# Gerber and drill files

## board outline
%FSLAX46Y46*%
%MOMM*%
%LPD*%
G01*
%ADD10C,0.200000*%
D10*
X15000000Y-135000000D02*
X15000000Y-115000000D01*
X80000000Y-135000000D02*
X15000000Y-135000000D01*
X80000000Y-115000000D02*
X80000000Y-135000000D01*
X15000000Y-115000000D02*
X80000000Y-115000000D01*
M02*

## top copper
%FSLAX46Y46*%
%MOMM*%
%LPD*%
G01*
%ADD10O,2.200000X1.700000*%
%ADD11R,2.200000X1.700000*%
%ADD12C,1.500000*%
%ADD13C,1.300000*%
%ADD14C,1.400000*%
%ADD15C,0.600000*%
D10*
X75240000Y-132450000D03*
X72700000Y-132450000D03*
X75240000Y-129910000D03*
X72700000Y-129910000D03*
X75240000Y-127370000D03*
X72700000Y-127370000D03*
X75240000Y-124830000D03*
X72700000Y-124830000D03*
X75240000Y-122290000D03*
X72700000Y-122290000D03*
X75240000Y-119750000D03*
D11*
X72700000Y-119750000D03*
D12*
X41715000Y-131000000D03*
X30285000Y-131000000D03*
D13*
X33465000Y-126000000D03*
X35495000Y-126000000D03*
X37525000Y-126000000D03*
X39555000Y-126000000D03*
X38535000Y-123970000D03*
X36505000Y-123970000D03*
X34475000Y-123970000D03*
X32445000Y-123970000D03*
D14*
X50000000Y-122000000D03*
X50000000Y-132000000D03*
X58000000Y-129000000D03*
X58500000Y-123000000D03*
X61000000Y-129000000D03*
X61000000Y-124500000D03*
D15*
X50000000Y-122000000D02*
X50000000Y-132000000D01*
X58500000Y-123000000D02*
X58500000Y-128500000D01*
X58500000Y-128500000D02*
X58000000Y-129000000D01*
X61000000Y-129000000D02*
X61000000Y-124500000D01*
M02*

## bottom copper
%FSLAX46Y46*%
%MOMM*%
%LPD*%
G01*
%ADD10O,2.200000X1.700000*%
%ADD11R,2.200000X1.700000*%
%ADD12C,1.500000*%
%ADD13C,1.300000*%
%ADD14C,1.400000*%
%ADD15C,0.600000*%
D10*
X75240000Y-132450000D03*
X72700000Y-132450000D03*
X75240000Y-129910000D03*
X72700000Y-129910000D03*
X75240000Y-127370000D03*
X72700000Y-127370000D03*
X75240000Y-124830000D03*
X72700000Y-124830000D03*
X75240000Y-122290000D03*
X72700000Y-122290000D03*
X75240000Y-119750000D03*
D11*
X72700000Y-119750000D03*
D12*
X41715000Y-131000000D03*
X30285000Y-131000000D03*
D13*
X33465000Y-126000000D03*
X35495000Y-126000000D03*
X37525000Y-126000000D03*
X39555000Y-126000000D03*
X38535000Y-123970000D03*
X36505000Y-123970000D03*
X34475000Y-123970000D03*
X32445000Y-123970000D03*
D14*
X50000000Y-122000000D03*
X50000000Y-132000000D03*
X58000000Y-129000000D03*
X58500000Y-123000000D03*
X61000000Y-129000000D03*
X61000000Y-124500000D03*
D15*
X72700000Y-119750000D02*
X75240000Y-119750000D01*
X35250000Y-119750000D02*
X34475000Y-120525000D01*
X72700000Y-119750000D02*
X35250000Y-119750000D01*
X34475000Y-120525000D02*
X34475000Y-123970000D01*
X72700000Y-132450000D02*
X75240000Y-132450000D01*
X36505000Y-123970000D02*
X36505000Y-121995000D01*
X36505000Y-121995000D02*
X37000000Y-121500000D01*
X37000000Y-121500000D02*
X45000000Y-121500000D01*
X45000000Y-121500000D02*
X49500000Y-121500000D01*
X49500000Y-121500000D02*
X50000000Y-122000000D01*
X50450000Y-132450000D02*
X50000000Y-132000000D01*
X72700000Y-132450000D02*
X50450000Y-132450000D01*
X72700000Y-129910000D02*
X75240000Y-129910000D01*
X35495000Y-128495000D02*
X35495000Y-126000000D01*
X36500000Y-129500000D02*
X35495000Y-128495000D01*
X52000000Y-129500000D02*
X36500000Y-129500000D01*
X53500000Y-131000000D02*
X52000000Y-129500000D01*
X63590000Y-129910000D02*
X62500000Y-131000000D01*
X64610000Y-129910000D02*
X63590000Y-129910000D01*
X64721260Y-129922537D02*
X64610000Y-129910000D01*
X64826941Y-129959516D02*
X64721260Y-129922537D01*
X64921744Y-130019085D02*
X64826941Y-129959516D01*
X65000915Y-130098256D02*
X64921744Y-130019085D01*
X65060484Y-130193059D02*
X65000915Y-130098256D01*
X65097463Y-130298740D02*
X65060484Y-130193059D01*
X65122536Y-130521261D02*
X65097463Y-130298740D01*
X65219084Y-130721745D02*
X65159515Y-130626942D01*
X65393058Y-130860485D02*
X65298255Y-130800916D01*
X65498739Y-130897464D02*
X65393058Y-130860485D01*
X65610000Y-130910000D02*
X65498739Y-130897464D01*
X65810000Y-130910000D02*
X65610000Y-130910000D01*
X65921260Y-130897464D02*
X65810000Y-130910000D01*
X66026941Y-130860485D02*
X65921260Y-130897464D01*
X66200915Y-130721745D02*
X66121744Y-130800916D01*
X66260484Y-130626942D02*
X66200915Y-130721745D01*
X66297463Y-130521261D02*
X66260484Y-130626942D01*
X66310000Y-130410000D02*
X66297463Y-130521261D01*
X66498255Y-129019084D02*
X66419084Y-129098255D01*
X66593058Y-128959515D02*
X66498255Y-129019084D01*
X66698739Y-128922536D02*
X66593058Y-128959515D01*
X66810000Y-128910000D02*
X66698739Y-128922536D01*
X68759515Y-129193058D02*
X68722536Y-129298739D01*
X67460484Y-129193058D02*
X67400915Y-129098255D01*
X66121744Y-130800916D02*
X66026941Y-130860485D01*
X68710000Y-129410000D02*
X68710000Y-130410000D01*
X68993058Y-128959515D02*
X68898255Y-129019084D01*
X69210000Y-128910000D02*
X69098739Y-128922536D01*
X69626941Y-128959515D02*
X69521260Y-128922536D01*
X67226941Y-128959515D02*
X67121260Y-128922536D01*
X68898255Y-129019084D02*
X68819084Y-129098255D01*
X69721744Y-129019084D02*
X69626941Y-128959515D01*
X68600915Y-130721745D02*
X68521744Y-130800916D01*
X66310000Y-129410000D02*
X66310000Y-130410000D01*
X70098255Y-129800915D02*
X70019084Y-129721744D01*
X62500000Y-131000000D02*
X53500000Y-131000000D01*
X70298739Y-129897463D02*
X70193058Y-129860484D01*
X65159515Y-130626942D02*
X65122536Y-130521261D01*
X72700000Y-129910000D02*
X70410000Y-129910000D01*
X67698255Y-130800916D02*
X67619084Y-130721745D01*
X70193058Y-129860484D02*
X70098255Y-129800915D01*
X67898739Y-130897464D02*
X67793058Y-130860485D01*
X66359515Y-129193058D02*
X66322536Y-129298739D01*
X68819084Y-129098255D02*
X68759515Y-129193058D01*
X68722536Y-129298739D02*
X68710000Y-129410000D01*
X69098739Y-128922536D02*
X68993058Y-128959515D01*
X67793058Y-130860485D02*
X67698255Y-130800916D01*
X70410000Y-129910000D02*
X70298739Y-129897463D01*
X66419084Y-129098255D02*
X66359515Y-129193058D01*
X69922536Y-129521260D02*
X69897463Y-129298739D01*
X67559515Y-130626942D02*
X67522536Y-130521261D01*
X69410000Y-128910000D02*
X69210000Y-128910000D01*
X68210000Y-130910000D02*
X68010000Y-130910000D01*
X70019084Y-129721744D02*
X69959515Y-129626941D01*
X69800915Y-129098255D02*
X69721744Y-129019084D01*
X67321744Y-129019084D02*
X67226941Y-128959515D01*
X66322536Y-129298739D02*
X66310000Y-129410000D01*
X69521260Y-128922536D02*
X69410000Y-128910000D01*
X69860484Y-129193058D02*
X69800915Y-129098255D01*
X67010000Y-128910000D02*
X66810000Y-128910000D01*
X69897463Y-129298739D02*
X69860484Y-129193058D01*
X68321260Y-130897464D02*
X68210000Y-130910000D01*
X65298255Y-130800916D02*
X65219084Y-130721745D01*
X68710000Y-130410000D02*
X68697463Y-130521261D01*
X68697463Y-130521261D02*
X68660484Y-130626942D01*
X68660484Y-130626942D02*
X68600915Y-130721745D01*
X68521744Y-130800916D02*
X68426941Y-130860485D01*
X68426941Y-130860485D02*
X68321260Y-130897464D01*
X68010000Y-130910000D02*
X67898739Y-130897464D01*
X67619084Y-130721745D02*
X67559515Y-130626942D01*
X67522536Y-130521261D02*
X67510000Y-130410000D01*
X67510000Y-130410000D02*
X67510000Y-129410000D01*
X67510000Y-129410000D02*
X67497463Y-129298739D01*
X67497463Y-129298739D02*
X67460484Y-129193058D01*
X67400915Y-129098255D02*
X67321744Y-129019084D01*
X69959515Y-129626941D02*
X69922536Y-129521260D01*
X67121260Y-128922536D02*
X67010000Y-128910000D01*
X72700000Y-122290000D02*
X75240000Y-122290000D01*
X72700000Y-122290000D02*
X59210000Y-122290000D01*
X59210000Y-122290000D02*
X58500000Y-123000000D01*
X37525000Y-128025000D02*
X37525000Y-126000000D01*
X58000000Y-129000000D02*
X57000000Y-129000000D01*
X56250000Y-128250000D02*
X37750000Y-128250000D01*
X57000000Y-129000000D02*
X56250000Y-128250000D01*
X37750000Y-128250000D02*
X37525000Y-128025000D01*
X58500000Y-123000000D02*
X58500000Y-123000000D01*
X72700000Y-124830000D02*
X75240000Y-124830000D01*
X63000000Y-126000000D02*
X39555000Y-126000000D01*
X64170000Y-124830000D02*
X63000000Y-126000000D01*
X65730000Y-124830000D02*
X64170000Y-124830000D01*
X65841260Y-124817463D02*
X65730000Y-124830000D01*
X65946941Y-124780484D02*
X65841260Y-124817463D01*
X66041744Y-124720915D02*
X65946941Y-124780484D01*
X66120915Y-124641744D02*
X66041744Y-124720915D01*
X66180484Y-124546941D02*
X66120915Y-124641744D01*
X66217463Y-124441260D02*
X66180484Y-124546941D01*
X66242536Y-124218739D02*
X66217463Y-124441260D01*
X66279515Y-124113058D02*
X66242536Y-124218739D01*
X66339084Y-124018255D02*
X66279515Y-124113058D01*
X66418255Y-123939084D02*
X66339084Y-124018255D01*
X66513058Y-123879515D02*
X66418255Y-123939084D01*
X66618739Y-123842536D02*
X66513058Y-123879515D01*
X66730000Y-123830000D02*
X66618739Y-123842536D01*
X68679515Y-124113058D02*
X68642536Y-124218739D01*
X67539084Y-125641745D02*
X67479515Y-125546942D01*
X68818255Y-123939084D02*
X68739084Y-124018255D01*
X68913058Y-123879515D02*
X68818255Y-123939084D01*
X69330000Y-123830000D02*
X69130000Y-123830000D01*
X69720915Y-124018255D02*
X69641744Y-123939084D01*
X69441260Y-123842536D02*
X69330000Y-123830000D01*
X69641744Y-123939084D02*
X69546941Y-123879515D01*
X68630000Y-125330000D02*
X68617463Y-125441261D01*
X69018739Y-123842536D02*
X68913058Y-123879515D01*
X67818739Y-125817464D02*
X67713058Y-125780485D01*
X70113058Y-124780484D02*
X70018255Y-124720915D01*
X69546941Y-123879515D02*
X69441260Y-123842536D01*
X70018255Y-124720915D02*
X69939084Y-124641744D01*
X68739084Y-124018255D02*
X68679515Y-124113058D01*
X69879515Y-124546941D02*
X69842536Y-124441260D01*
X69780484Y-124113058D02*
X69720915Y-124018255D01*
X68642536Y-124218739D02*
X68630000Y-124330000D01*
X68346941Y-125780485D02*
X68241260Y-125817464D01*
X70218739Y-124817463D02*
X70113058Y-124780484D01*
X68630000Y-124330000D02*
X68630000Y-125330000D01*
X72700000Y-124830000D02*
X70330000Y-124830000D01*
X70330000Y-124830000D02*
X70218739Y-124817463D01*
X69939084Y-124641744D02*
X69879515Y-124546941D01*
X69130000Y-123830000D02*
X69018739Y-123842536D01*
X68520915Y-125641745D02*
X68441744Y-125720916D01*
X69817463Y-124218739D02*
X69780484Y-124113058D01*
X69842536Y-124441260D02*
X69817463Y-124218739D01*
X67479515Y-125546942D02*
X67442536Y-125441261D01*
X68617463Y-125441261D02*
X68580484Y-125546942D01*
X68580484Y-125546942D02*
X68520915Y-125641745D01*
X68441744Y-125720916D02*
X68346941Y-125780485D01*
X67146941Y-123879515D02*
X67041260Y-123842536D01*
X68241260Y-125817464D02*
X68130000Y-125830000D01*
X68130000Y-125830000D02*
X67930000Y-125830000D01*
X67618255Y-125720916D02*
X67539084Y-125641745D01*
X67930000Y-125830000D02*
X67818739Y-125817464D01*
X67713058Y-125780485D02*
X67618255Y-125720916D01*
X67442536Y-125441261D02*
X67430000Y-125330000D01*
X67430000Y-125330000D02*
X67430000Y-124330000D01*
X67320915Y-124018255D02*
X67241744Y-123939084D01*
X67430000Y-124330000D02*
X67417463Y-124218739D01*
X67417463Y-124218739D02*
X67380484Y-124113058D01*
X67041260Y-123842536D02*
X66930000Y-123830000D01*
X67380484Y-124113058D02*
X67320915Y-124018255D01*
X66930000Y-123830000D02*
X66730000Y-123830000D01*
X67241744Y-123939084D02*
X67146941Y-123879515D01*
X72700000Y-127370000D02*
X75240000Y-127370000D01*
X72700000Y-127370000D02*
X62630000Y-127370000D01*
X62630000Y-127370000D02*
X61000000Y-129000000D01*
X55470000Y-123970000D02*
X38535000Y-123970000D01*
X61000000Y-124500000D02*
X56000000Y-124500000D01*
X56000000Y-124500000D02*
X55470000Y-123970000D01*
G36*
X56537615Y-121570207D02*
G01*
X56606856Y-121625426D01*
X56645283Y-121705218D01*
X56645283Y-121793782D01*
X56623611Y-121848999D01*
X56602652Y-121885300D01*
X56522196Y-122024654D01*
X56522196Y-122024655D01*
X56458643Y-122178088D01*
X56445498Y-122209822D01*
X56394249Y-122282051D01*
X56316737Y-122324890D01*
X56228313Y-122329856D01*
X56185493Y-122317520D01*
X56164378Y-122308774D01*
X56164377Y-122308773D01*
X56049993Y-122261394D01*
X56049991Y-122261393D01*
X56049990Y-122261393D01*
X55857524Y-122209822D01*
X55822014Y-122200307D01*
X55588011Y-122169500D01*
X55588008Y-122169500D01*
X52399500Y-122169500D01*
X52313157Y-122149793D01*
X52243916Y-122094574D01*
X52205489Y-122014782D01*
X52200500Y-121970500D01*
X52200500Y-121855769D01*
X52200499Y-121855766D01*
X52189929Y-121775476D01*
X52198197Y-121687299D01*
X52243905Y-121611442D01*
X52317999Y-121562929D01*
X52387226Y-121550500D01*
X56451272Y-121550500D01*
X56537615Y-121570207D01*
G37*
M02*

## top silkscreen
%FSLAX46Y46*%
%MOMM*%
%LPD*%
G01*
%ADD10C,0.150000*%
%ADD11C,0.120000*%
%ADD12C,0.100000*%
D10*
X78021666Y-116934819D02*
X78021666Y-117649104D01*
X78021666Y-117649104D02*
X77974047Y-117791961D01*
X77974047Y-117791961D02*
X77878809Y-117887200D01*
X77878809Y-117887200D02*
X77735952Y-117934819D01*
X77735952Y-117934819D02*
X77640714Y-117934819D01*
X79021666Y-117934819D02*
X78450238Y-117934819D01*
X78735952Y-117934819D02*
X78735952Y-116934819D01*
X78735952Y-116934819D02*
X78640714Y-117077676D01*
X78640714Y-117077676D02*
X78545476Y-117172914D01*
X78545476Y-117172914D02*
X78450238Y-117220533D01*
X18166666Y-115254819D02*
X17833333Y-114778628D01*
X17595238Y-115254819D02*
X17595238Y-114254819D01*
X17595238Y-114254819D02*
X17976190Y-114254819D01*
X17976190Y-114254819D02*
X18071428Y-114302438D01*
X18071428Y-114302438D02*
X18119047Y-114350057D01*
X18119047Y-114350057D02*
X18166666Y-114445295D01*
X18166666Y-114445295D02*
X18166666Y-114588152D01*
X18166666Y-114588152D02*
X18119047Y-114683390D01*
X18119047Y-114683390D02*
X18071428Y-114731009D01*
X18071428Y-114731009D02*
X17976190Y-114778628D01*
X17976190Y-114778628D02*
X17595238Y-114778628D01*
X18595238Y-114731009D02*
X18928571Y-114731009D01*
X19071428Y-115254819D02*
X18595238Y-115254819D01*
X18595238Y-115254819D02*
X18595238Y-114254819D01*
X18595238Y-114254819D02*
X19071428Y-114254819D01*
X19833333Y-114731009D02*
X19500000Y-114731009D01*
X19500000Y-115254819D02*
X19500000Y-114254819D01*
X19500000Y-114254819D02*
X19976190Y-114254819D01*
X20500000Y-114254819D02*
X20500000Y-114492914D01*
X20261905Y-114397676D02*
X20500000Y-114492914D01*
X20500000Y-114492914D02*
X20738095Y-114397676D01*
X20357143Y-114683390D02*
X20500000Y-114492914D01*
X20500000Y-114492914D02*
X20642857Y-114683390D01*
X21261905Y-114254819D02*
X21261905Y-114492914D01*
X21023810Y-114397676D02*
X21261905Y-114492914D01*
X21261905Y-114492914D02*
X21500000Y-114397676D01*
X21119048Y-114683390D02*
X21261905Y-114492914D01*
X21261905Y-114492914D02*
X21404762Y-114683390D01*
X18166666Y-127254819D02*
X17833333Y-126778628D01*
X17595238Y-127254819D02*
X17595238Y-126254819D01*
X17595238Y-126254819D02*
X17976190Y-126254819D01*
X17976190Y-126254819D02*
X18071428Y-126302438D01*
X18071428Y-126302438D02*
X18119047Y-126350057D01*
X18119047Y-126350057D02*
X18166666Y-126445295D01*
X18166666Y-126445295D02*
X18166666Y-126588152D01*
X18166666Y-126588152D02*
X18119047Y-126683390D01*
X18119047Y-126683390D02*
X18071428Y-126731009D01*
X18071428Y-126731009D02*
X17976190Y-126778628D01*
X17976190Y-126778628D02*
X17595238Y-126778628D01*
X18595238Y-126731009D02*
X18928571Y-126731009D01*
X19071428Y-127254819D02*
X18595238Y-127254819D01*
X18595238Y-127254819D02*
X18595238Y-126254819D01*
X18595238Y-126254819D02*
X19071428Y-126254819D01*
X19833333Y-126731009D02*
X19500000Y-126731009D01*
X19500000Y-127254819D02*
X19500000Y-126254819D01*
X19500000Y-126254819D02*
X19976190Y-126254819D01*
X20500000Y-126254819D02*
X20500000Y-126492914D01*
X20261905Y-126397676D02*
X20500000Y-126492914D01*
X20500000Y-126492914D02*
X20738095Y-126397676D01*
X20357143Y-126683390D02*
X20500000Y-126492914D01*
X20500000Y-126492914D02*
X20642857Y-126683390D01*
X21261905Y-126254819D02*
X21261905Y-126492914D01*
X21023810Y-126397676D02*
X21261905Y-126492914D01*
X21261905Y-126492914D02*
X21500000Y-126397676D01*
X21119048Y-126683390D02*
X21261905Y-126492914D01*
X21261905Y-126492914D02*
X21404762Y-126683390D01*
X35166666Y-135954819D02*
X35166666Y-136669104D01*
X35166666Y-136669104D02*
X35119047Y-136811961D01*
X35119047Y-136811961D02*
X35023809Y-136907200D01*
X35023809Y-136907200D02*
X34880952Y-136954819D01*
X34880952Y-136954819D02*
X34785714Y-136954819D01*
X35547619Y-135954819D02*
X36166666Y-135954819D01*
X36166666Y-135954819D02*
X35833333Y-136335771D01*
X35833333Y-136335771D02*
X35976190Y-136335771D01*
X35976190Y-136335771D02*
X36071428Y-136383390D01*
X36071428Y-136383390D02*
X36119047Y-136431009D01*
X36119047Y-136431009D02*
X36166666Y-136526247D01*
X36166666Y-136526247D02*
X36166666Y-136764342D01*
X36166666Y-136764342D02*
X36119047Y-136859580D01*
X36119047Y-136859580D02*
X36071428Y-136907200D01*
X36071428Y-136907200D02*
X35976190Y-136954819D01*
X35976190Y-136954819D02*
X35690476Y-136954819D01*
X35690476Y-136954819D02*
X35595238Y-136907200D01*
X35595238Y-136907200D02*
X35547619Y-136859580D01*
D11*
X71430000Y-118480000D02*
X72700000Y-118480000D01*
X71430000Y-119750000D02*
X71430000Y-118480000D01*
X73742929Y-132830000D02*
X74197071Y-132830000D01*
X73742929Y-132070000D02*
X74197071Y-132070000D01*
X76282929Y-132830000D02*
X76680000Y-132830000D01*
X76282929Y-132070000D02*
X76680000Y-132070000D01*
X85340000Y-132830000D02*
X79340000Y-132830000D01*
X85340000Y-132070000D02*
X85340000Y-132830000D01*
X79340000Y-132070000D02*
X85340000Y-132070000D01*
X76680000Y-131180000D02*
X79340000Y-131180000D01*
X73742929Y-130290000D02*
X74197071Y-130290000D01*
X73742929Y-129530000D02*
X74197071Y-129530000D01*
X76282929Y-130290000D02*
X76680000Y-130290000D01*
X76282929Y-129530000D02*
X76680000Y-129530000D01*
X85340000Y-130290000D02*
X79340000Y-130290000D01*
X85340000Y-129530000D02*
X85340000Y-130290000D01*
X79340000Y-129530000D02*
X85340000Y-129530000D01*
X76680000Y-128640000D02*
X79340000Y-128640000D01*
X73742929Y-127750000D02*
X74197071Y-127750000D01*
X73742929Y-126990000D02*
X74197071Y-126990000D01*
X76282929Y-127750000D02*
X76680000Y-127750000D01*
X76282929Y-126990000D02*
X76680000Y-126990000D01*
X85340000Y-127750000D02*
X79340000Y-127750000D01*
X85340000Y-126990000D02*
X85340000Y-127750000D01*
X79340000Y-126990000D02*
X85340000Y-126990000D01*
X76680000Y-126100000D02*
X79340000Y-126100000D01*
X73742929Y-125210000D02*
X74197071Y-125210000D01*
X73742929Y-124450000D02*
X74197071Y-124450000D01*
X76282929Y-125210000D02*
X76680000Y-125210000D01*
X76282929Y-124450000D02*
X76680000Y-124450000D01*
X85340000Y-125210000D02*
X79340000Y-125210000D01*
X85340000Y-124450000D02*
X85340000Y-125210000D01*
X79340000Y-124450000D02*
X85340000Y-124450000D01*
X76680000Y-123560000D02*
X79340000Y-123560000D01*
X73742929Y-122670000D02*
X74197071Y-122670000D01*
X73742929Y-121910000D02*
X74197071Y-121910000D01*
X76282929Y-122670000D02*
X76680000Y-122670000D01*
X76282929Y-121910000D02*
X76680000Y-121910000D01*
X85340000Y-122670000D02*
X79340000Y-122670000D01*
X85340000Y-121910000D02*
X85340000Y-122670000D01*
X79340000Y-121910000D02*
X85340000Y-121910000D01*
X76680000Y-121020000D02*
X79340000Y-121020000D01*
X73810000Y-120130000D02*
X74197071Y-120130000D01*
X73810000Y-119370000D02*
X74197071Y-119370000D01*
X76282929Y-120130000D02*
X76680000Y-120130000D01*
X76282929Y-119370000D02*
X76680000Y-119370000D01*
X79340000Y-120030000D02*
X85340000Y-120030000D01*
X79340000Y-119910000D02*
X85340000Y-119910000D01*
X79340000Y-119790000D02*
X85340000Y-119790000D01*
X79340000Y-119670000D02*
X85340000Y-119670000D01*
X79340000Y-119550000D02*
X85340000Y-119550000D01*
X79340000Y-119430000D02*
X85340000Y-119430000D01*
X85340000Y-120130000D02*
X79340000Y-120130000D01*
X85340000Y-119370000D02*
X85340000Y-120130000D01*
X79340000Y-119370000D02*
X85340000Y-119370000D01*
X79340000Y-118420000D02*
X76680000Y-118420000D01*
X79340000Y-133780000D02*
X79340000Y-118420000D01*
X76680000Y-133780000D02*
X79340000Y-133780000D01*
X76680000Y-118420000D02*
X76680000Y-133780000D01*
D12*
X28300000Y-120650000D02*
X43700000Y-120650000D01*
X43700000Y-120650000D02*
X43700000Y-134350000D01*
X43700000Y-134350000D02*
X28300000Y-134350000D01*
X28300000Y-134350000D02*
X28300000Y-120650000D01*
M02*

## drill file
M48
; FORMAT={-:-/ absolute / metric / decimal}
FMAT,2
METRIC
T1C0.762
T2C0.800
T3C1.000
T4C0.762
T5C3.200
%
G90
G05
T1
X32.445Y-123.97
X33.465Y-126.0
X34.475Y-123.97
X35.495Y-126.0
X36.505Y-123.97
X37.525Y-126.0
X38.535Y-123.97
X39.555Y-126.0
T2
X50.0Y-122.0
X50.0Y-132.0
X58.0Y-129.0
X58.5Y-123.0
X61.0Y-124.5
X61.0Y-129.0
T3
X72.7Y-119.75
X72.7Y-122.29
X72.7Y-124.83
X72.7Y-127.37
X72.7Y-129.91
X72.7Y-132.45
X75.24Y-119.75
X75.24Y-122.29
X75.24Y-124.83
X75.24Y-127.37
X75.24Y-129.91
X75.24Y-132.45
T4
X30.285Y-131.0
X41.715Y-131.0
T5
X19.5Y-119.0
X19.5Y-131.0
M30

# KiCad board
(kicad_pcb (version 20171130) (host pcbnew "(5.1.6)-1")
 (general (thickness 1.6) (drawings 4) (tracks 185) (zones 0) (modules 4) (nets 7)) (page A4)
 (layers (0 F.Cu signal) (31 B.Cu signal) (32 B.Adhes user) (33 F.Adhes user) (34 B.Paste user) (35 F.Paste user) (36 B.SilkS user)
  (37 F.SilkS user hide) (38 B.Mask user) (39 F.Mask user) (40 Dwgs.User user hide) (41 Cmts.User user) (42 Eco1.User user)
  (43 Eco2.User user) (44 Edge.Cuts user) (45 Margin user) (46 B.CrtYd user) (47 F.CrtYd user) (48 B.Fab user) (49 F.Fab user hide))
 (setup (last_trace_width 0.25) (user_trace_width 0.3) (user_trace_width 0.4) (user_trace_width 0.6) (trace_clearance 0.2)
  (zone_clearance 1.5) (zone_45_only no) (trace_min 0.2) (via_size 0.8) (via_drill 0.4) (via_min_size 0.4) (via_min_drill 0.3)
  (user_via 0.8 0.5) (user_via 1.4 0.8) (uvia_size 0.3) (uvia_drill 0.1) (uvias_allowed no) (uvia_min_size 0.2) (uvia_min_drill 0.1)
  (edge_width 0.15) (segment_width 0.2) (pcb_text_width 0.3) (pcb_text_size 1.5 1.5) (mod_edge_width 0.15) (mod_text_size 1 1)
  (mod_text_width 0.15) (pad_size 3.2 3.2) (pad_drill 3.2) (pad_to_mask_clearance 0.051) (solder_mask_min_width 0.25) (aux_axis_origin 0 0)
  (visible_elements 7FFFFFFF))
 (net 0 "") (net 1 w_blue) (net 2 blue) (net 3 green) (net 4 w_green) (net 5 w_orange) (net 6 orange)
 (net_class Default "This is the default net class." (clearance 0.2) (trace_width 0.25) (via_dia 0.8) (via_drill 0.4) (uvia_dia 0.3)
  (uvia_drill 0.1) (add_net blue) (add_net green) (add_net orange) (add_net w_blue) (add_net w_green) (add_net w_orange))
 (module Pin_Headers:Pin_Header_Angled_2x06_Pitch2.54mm (layer F.Cu) (at 72.7 119.75)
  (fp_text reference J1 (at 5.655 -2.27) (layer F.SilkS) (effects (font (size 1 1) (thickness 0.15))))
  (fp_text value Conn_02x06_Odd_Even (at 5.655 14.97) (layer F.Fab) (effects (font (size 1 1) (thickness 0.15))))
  (fp_line (start -1.27 -1.27) (end 0 -1.27) (layer F.SilkS) (width 0.12))
  (fp_line (start -1.27 0) (end -1.27 -1.27) (layer F.SilkS) (width 0.12))
  (fp_line (start 1.042929 13.08) (end 1.497071 13.08) (layer F.SilkS) (width 0.12))
  (fp_line (start 1.042929 12.32) (end 1.497071 12.32) (layer F.SilkS) (width 0.12))
  (fp_line (start 3.582929 13.08) (end 3.98 13.08) (layer F.SilkS) (width 0.12))
  (fp_line (start 3.582929 12.32) (end 3.98 12.32) (layer F.SilkS) (width 0.12))
  (fp_line (start 12.64 13.08) (end 6.64 13.08) (layer F.SilkS) (width 0.12))
  (fp_line (start 12.64 12.32) (end 12.64 13.08) (layer F.SilkS) (width 0.12))
  (fp_line (start 6.64 12.32) (end 12.64 12.32) (layer F.SilkS) (width 0.12))
  (fp_line (start 3.98 11.43) (end 6.64 11.43) (layer F.SilkS) (width 0.12))
  (fp_line (start 1.042929 10.54) (end 1.497071 10.54) (layer F.SilkS) (width 0.12))
  (fp_line (start 1.042929 9.78) (end 1.497071 9.78) (layer F.SilkS) (width 0.12))
  (fp_line (start 3.582929 10.54) (end 3.98 10.54) (layer F.SilkS) (width 0.12))
  (fp_line (start 3.582929 9.78) (end 3.98 9.78) (layer F.SilkS) (width 0.12))
  (fp_line (start 12.64 10.54) (end 6.64 10.54) (layer F.SilkS) (width 0.12))
  (fp_line (start 12.64 9.78) (end 12.64 10.54) (layer F.SilkS) (width 0.12))
  (fp_line (start 6.64 9.78) (end 12.64 9.78) (layer F.SilkS) (width 0.12))
  (fp_line (start 3.98 8.89) (end 6.64 8.89) (layer F.SilkS) (width 0.12))
  (fp_line (start 1.042929 8) (end 1.497071 8) (layer F.SilkS) (width 0.12))
  (fp_line (start 1.042929 7.24) (end 1.497071 7.24) (layer F.SilkS) (width 0.12))
  (fp_line (start 3.582929 8) (end 3.98 8) (layer F.SilkS) (width 0.12))
  (fp_line (start 3.582929 7.24) (end 3.98 7.24) (layer F.SilkS) (width 0.12))
  (fp_line (start 12.64 8) (end 6.64 8) (layer F.SilkS) (width 0.12))
  (fp_line (start 12.64 7.24) (end 12.64 8) (layer F.SilkS) (width 0.12))
  (fp_line (start 6.64 7.24) (end 12.64 7.24) (layer F.SilkS) (width 0.12))
  (fp_line (start 3.98 6.35) (end 6.64 6.35) (layer F.SilkS) (width 0.12))
  (fp_line (start 1.042929 5.46) (end 1.497071 5.46) (layer F.SilkS) (width 0.12))
  (fp_line (start 1.042929 4.7) (end 1.497071 4.7) (layer F.SilkS) (width 0.12))
  (fp_line (start 3.582929 5.46) (end 3.98 5.46) (layer F.SilkS) (width 0.12))
  (fp_line (start 3.582929 4.7) (end 3.98 4.7) (layer F.SilkS) (width 0.12))
  (fp_line (start 12.64 5.46) (end 6.64 5.46) (layer F.SilkS) (width 0.12))
  (fp_line (start 12.64 4.7) (end 12.64 5.46) (layer F.SilkS) (width 0.12))
  (fp_line (start 6.64 4.7) (end 12.64 4.7) (layer F.SilkS) (width 0.12))
  (fp_line (start 3.98 3.81) (end 6.64 3.81) (layer F.SilkS) (width 0.12))
  (fp_line (start 1.042929 2.92) (end 1.497071 2.92) (layer F.SilkS) (width 0.12))
  (fp_line (start 1.042929 2.16) (end 1.497071 2.16) (layer F.SilkS) (width 0.12))
  (fp_line (start 3.582929 2.92) (end 3.98 2.92) (layer F.SilkS) (width 0.12))
  (fp_line (start 3.582929 2.16) (end 3.98 2.16) (layer F.SilkS) (width 0.12))
  (fp_line (start 12.64 2.92) (end 6.64 2.92) (layer F.SilkS) (width 0.12))
  (fp_line (start 12.64 2.16) (end 12.64 2.92) (layer F.SilkS) (width 0.12))
  (fp_line (start 6.64 2.16) (end 12.64 2.16) (layer F.SilkS) (width 0.12))
  (fp_line (start 3.98 1.27) (end 6.64 1.27) (layer F.SilkS) (width 0.12))
  (fp_line (start 1.11 0.38) (end 1.497071 0.38) (layer F.SilkS) (width 0.12))
  (fp_line (start 1.11 -0.38) (end 1.497071 -0.38) (layer F.SilkS) (width 0.12))
  (fp_line (start 3.582929 0.38) (end 3.98 0.38) (layer F.SilkS) (width 0.12))
  (fp_line (start 3.582929 -0.38) (end 3.98 -0.38) (layer F.SilkS) (width 0.12))
  (fp_line (start 6.64 0.28) (end 12.64 0.28) (layer F.SilkS) (width 0.12))
  (fp_line (start 6.64 0.16) (end 12.64 0.16) (layer F.SilkS) (width 0.12))
  (fp_line (start 6.64 0.04) (end 12.64 0.04) (layer F.SilkS) (width 0.12))
  (fp_line (start 6.64 -0.08) (end 12.64 -0.08) (layer F.SilkS) (width 0.12))
  (fp_line (start 6.64 -0.2) (end 12.64 -0.2) (layer F.SilkS) (width 0.12))
  (fp_line (start 6.64 -0.32) (end 12.64 -0.32) (layer F.SilkS) (width 0.12))
  (fp_line (start 12.64 0.38) (end 6.64 0.38) (layer F.SilkS) (width 0.12))
  (fp_line (start 12.64 -0.38) (end 12.64 0.38) (layer F.SilkS) (width 0.12))
  (fp_line (start 6.64 -0.38) (end 12.64 -0.38) (layer F.SilkS) (width 0.12))
  (fp_line (start 6.64 -1.33) (end 3.98 -1.33) (layer F.SilkS) (width 0.12))
  (fp_line (start 6.64 14.03) (end 6.64 -1.33) (layer F.SilkS) (width 0.12))
  (fp_line (start 3.98 14.03) (end 6.64 14.03) (layer F.SilkS) (width 0.12))
  (fp_line (start 3.98 -1.33) (end 3.98 14.03) (layer F.SilkS) (width 0.12))
  (pad 12 thru_hole oval (at 2.54 12.7) (size 2.2 1.7) (drill 1) (layers *.Cu *.Mask) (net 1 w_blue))
  (pad 11 thru_hole oval (at 0 12.7) (size 2.2 1.7) (drill 1) (layers *.Cu *.Mask) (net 1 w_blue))
  (pad 10 thru_hole oval (at 2.54 10.16) (size 2.2 1.7) (drill 1) (layers *.Cu *.Mask) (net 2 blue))
  (pad 9 thru_hole oval (at 0 10.16) (size 2.2 1.7) (drill 1) (layers *.Cu *.Mask) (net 2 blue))
  (pad 8 thru_hole oval (at 2.54 7.62) (size 2.2 1.7) (drill 1) (layers *.Cu *.Mask) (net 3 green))
  (pad 7 thru_hole oval (at 0 7.62) (size 2.2 1.7) (drill 1) (layers *.Cu *.Mask) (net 3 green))
  (pad 6 thru_hole oval (at 2.54 5.08) (size 2.2 1.7) (drill 1) (layers *.Cu *.Mask) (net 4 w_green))
  (pad 5 thru_hole oval (at 0 5.08) (size 2.2 1.7) (drill 1) (layers *.Cu *.Mask) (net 4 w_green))
  (pad 4 thru_hole oval (at 2.54 2.54) (size 2.2 1.7) (drill 1) (layers *.Cu *.Mask) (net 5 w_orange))
  (pad 3 thru_hole oval (at 0 2.54) (size 2.2 1.7) (drill 1) (layers *.Cu *.Mask) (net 5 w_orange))
  (pad 2 thru_hole oval (at 2.54 0) (size 2.2 1.7) (drill 1) (layers *.Cu *.Mask) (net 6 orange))
  (pad 1 thru_hole rect (at 0 0) (size 2.2 1.7) (drill 1) (layers *.Cu *.Mask) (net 6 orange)))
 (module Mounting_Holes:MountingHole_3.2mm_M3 (layer F.Cu) (at 19.5 119)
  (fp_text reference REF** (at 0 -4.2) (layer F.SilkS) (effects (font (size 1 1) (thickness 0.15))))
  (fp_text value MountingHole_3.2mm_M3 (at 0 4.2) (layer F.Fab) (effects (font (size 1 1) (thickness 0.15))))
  (pad "" np_thru_hole circle (at 0 0) (size 3.2 3.2) (drill 3.2) (layers *.Cu *.Mask)))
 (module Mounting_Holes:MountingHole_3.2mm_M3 (layer F.Cu) (at 19.5 131)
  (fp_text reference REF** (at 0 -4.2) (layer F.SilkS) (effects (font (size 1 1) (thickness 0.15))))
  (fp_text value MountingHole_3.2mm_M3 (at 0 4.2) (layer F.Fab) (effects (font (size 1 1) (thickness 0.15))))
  (pad 1 np_thru_hole circle (at 0 0) (size 3.2 3.2) (drill 3.2) (layers *.Cu *.Mask)))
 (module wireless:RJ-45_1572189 (layer F.Cu) (at 36 126)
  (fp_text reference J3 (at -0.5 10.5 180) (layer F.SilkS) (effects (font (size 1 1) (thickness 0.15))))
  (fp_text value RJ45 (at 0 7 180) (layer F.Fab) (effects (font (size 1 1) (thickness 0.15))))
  (fp_line (start -7.7 -5.35) (end 7.7 -5.35) (layer F.SilkS) (width 0.1))
  (fp_line (start 7.7 -5.35) (end 7.7 8.35) (layer F.SilkS) (width 0.1))
  (fp_line (start 7.7 8.35) (end -7.7 8.35) (layer F.SilkS) (width 0.1))
  (fp_line (start -7.7 8.35) (end -7.7 -5.35) (layer F.SilkS) (width 0.1))
  (pad "" np_thru_hole circle (at 5.715 5) (size 1.5 1.5) (drill 0.762) (layers *.Cu *.Mask))
  (pad "" np_thru_hole circle (at -5.715 5) (size 1.5 1.5) (drill 0.762) (layers *.Cu *.Mask))
  (pad 8 thru_hole circle (at -2.535 0) (size 1.3 1.3) (drill 0.762) (layers *.Cu *.Mask))
  (pad 4 thru_hole circle (at -0.505 0) (size 1.3 1.3) (drill 0.762) (layers *.Cu *.Mask) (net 2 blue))
  (pad 3 thru_hole circle (at 1.525 0) (size 1.3 1.3) (drill 0.762) (layers *.Cu *.Mask) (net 5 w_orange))
  (pad 2 thru_hole circle (at 3.555 0) (size 1.3 1.3) (drill 0.762) (layers *.Cu *.Mask) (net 4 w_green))
  (pad 1 thru_hole circle (at 2.535 -2.03) (size 1.3 1.3) (drill 0.762) (layers *.Cu *.Mask) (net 3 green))
  (pad 5 thru_hole circle (at 0.505 -2.03) (size 1.3 1.3) (drill 0.762) (layers *.Cu *.Mask) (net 1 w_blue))
  (pad 6 thru_hole circle (at -1.525 -2.03) (size 1.3 1.3) (drill 0.762) (layers *.Cu *.Mask) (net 6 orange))
  (pad 7 thru_hole circle (at -3.555 -2.03) (size 1.3 1.3) (drill 0.762) (layers *.Cu *.Mask)))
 (gr_line (start 15 135) (end 15 115) (layer Edge.Cuts) (width 0.2))
 (gr_line (start 80 135) (end 15 135) (layer Edge.Cuts) (width 0.2))
 (gr_line (start 80 115) (end 80 135) (layer Edge.Cuts) (width 0.2))
 (gr_line (start 15 115) (end 80 115) (layer Edge.Cuts) (width 0.2))
 (segment (start 72.7 119.75) (end 75.24 119.75) (width 0.6) (layer B.Cu) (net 6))
 (segment (start 35.25 119.75) (end 34.475 120.525) (width 0.6) (layer B.Cu) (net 6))
 (segment (start 72.7 119.75) (end 35.25 119.75) (width 0.6) (layer B.Cu) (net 6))
 (segment (start 34.475 120.525) (end 34.475 123.97) (width 0.6) (layer B.Cu) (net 6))
 (segment (start 72.7 132.45) (end 75.24 132.45) (width 0.6) (layer B.Cu) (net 1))
 (segment (start 36.505 123.97) (end 36.505 121.995) (width 0.6) (layer B.Cu) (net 1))
 (segment (start 36.505 121.995) (end 37 121.5) (width 0.6) (layer B.Cu) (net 1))
 (segment (start 37 121.5) (end 45 121.5) (width 0.6) (layer B.Cu) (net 1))
 (segment (start 45 121.5) (end 49.5 121.5) (width 0.6) (layer B.Cu) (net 1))
 (via (at 50 122) (size 1.4) (drill 0.8) (layers F.Cu B.Cu) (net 1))
 (segment (start 49.5 121.5) (end 50 122) (width 0.6) (layer B.Cu) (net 1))
 (segment (start 50 122) (end 50 132) (width 0.6) (layer F.Cu) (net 1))
 (via (at 50 132) (size 1.4) (drill 0.8) (layers F.Cu B.Cu) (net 1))
 (segment (start 50.45 132.45) (end 50 132) (width 0.6) (layer B.Cu) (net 1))
 (segment (start 72.7 132.45) (end 50.45 132.45) (width 0.6) (layer B.Cu) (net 1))
 (segment (start 72.7 129.91) (end 75.24 129.91) (width 0.6) (layer B.Cu) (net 2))
 (segment (start 35.495 128.495) (end 35.495 126) (width 0.6) (layer B.Cu) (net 2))
 (segment (start 36.5 129.5) (end 35.495 128.495) (width 0.6) (layer B.Cu) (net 2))
 (segment (start 52 129.5) (end 36.5 129.5) (width 0.6) (layer B.Cu) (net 2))
 (segment (start 53.5 131) (end 52 129.5) (width 0.6) (layer B.Cu) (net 2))
 (segment (start 63.59 129.91) (end 62.5 131) (width 0.6) (layer B.Cu) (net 2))
 (segment (start 64.61 129.91) (end 63.59 129.91) (width 0.6) (layer B.Cu) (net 2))
 (segment (start 64.72126 129.922537) (end 64.61 129.91) (width 0.6) (layer B.Cu) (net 2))
 (segment (start 64.826941 129.959516) (end 64.72126 129.922537) (width 0.6) (layer B.Cu) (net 2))
 (segment (start 64.921744 130.019085) (end 64.826941 129.959516) (width 0.6) (layer B.Cu) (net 2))
 (segment (start 65.000915 130.098256) (end 64.921744 130.019085) (width 0.6) (layer B.Cu) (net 2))
 (segment (start 65.060484 130.193059) (end 65.000915 130.098256) (width 0.6) (layer B.Cu) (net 2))
 (segment (start 65.097463 130.29874) (end 65.060484 130.193059) (width 0.6) (layer B.Cu) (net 2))
 (segment (start 65.122536 130.521261) (end 65.097463 130.29874) (width 0.6) (layer B.Cu) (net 2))
 (segment (start 65.219084 130.721745) (end 65.159515 130.626942) (width 0.6) (layer B.Cu) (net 2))
 (segment (start 65.393058 130.860485) (end 65.298255 130.800916) (width 0.6) (layer B.Cu) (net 2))
 (segment (start 65.498739 130.897464) (end 65.393058 130.860485) (width 0.6) (layer B.Cu) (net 2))
 (segment (start 65.61 130.91) (end 65.498739 130.897464) (width 0.6) (layer B.Cu) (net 2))
 (segment (start 65.81 130.91) (end 65.61 130.91) (width 0.6) (layer B.Cu) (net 2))
 (segment (start 65.92126 130.897464) (end 65.81 130.91) (width 0.6) (layer B.Cu) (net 2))
 (segment (start 66.026941 130.860485) (end 65.92126 130.897464) (width 0.6) (layer B.Cu) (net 2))
 (segment (start 66.200915 130.721745) (end 66.121744 130.800916) (width 0.6) (layer B.Cu) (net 2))
 (segment (start 66.260484 130.626942) (end 66.200915 130.721745) (width 0.6) (layer B.Cu) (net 2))
 (segment (start 66.297463 130.521261) (end 66.260484 130.626942) (width 0.6) (layer B.Cu) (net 2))
 (segment (start 66.31 130.41) (end 66.297463 130.521261) (width 0.6) (layer B.Cu) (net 2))
 (segment (start 66.498255 129.019084) (end 66.419084 129.098255) (width 0.6) (layer B.Cu) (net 2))
 (segment (start 66.593058 128.959515) (end 66.498255 129.019084) (width 0.6) (layer B.Cu) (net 2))
 (segment (start 66.698739 128.922536) (end 66.593058 128.959515) (width 0.6) (layer B.Cu) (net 2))
 (segment (start 66.81 128.91) (end 66.698739 128.922536) (width 0.6) (layer B.Cu) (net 2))
 (segment (start 68.759515 129.193058) (end 68.722536 129.298739) (width 0.6) (layer B.Cu) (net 2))
 (segment (start 67.460484 129.193058) (end 67.400915 129.098255) (width 0.6) (layer B.Cu) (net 2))
 (segment (start 66.121744 130.800916) (end 66.026941 130.860485) (width 0.6) (layer B.Cu) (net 2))
 (segment (start 68.71 129.41) (end 68.71 130.41) (width 0.6) (layer B.Cu) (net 2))
 (segment (start 68.993058 128.959515) (end 68.898255 129.019084) (width 0.6) (layer B.Cu) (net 2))
 (segment (start 69.21 128.91) (end 69.098739 128.922536) (width 0.6) (layer B.Cu) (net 2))
 (segment (start 69.626941 128.959515) (end 69.52126 128.922536) (width 0.6) (layer B.Cu) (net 2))
 (segment (start 67.226941 128.959515) (end 67.12126 128.922536) (width 0.6) (layer B.Cu) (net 2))
 (segment (start 68.898255 129.019084) (end 68.819084 129.098255) (width 0.6) (layer B.Cu) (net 2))
 (segment (start 69.721744 129.019084) (end 69.626941 128.959515) (width 0.6) (layer B.Cu) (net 2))
 (segment (start 68.600915 130.721745) (end 68.521744 130.800916) (width 0.6) (layer B.Cu) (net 2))
 (segment (start 66.31 129.41) (end 66.31 130.41) (width 0.6) (layer B.Cu) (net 2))
 (segment (start 70.098255 129.800915) (end 70.019084 129.721744) (width 0.6) (layer B.Cu) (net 2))
 (segment (start 62.5 131) (end 53.5 131) (width 0.6) (layer B.Cu) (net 2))
 (segment (start 70.298739 129.897463) (end 70.193058 129.860484) (width 0.6) (layer B.Cu) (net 2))
 (segment (start 65.159515 130.626942) (end 65.122536 130.521261) (width 0.6) (layer B.Cu) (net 2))
 (segment (start 72.7 129.91) (end 70.41 129.91) (width 0.6) (layer B.Cu) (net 2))
 (segment (start 67.698255 130.800916) (end 67.619084 130.721745) (width 0.6) (layer B.Cu) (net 2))
 (segment (start 70.193058 129.860484) (end 70.098255 129.800915) (width 0.6) (layer B.Cu) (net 2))
 (segment (start 67.898739 130.897464) (end 67.793058 130.860485) (width 0.6) (layer B.Cu) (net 2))
 (segment (start 66.359515 129.193058) (end 66.322536 129.298739) (width 0.6) (layer B.Cu) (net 2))
 (segment (start 68.819084 129.098255) (end 68.759515 129.193058) (width 0.6) (layer B.Cu) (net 2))
 (segment (start 68.722536 129.298739) (end 68.71 129.41) (width 0.6) (layer B.Cu) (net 2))
 (segment (start 69.098739 128.922536) (end 68.993058 128.959515) (width 0.6) (layer B.Cu) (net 2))
 (segment (start 67.793058 130.860485) (end 67.698255 130.800916) (width 0.6) (layer B.Cu) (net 2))
 (segment (start 70.41 129.91) (end 70.298739 129.897463) (width 0.6) (layer B.Cu) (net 2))
 (segment (start 66.419084 129.098255) (end 66.359515 129.193058) (width 0.6) (layer B.Cu) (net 2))
 (segment (start 69.922536 129.52126) (end 69.897463 129.298739) (width 0.6) (layer B.Cu) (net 2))
 (segment (start 67.559515 130.626942) (end 67.522536 130.521261) (width 0.6) (layer B.Cu) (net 2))
 (segment (start 69.41 128.91) (end 69.21 128.91) (width 0.6) (layer B.Cu) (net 2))
 (segment (start 68.21 130.91) (end 68.01 130.91) (width 0.6) (layer B.Cu) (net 2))
 (segment (start 70.019084 129.721744) (end 69.959515 129.626941) (width 0.6) (layer B.Cu) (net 2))
 (segment (start 69.800915 129.098255) (end 69.721744 129.019084) (width 0.6) (layer B.Cu) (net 2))
 (segment (start 67.321744 129.019084) (end 67.226941 128.959515) (width 0.6) (layer B.Cu) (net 2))
 (segment (start 66.322536 129.298739) (end 66.31 129.41) (width 0.6) (layer B.Cu) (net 2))
 (segment (start 69.52126 128.922536) (end 69.41 128.91) (width 0.6) (layer B.Cu) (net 2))
 (segment (start 69.860484 129.193058) (end 69.800915 129.098255) (width 0.6) (layer B.Cu) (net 2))
 (segment (start 67.01 128.91) (end 66.81 128.91) (width 0.6) (layer B.Cu) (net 2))
 (segment (start 69.897463 129.298739) (end 69.860484 129.193058) (width 0.6) (layer B.Cu) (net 2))
 (segment (start 68.32126 130.897464) (end 68.21 130.91) (width 0.6) (layer B.Cu) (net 2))
 (segment (start 65.298255 130.800916) (end 65.219084 130.721745) (width 0.6) (layer B.Cu) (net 2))
 (segment (start 68.71 130.41) (end 68.697463 130.521261) (width 0.6) (layer B.Cu) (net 2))
 (segment (start 68.697463 130.521261) (end 68.660484 130.626942) (width 0.6) (layer B.Cu) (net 2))
 (segment (start 68.660484 130.626942) (end 68.600915 130.721745) (width 0.6) (layer B.Cu) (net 2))
 (segment (start 68.521744 130.800916) (end 68.426941 130.860485) (width 0.6) (layer B.Cu) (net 2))
 (segment (start 68.426941 130.860485) (end 68.32126 130.897464) (width 0.6) (layer B.Cu) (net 2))
 (segment (start 68.01 130.91) (end 67.898739 130.897464) (width 0.6) (layer B.Cu) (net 2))
 (segment (start 67.619084 130.721745) (end 67.559515 130.626942) (width 0.6) (layer B.Cu) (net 2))
 (segment (start 67.522536 130.521261) (end 67.51 130.41) (width 0.6) (layer B.Cu) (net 2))
 (segment (start 67.51 130.41) (end 67.51 129.41) (width 0.6) (layer B.Cu) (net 2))
 (segment (start 67.51 129.41) (end 67.497463 129.298739) (width 0.6) (layer B.Cu) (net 2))
 (segment (start 67.497463 129.298739) (end 67.460484 129.193058) (width 0.6) (layer B.Cu) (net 2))
 (segment (start 67.400915 129.098255) (end 67.321744 129.019084) (width 0.6) (layer B.Cu) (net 2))
 (segment (start 69.959515 129.626941) (end 69.922536 129.52126) (width 0.6) (layer B.Cu) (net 2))
 (segment (start 67.12126 128.922536) (end 67.01 128.91) (width 0.6) (layer B.Cu) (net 2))
 (segment (start 72.7 122.29) (end 75.24 122.29) (width 0.6) (layer B.Cu) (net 5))
 (segment (start 72.7 122.29) (end 59.21 122.29) (width 0.6) (layer B.Cu) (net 5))
 (segment (start 59.21 122.29) (end 58.5 123) (width 0.6) (layer B.Cu) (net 5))
 (segment (start 58.5 123) (end 58.5 128.5) (width 0.6) (layer F.Cu) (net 5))
 (segment (start 58.5 128.5) (end 58 129) (width 0.6) (layer F.Cu) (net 5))
 (via (at 58 129) (size 1.4) (drill 0.8) (layers F.Cu B.Cu) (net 5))
 (segment (start 37.525 128.025) (end 37.525 126) (width 0.6) (layer B.Cu) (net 5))
 (segment (start 58 129) (end 57 129) (width 0.6) (layer B.Cu) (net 5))
 (segment (start 56.25 128.25) (end 37.75 128.25) (width 0.6) (layer B.Cu) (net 5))
 (segment (start 57 129) (end 56.25 128.25) (width 0.6) (layer B.Cu) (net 5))
 (segment (start 37.75 128.25) (end 37.525 128.025) (width 0.6) (layer B.Cu) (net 5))
 (segment (start 58.5 123) (end 58.5 123) (width 0.6) (layer B.Cu) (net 5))
 (via (at 58.5 123) (size 1.4) (drill 0.8) (layers F.Cu B.Cu) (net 5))
 (segment (start 72.7 124.83) (end 75.24 124.83) (width 0.6) (layer B.Cu) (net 4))
 (segment (start 63 126) (end 39.555 126) (width 0.6) (layer B.Cu) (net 4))
 (segment (start 64.17 124.83) (end 63 126) (width 0.6) (layer B.Cu) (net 4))
 (segment (start 65.73 124.83) (end 64.17 124.83) (width 0.6) (layer B.Cu) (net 4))
 (segment (start 65.84126 124.817463) (end 65.73 124.83) (width 0.6) (layer B.Cu) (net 4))
 (segment (start 65.946941 124.780484) (end 65.84126 124.817463) (width 0.6) (layer B.Cu) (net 4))
 (segment (start 66.041744 124.720915) (end 65.946941 124.780484) (width 0.6) (layer B.Cu) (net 4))
 (segment (start 66.120915 124.641744) (end 66.041744 124.720915) (width 0.6) (layer B.Cu) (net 4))
 (segment (start 66.180484 124.546941) (end 66.120915 124.641744) (width 0.6) (layer B.Cu) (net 4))
 (segment (start 66.217463 124.44126) (end 66.180484 124.546941) (width 0.6) (layer B.Cu) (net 4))
 (segment (start 66.242536 124.218739) (end 66.217463 124.44126) (width 0.6) (layer B.Cu) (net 4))
 (segment (start 66.279515 124.113058) (end 66.242536 124.218739) (width 0.6) (layer B.Cu) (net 4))
 (segment (start 66.339084 124.018255) (end 66.279515 124.113058) (width 0.6) (layer B.Cu) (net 4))
 (segment (start 66.418255 123.939084) (end 66.339084 124.018255) (width 0.6) (layer B.Cu) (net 4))
 (segment (start 66.513058 123.879515) (end 66.418255 123.939084) (width 0.6) (layer B.Cu) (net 4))
 (segment (start 66.618739 123.842536) (end 66.513058 123.879515) (width 0.6) (layer B.Cu) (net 4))
 (segment (start 66.73 123.83) (end 66.618739 123.842536) (width 0.6) (layer B.Cu) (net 4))
 (segment (start 68.679515 124.113058) (end 68.642536 124.218739) (width 0.6) (layer B.Cu) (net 4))
 (segment (start 67.539084 125.641745) (end 67.479515 125.546942) (width 0.6) (layer B.Cu) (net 4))
 (segment (start 68.818255 123.939084) (end 68.739084 124.018255) (width 0.6) (layer B.Cu) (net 4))
 (segment (start 68.913058 123.879515) (end 68.818255 123.939084) (width 0.6) (layer B.Cu) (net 4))
 (segment (start 69.33 123.83) (end 69.13 123.83) (width 0.6) (layer B.Cu) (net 4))
 (segment (start 69.720915 124.018255) (end 69.641744 123.939084) (width 0.6) (layer B.Cu) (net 4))
 (segment (start 69.44126 123.842536) (end 69.33 123.83) (width 0.6) (layer B.Cu) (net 4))
 (segment (start 69.641744 123.939084) (end 69.546941 123.879515) (width 0.6) (layer B.Cu) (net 4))
 (segment (start 68.63 125.33) (end 68.617463 125.441261) (width 0.6) (layer B.Cu) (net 4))
 (segment (start 69.018739 123.842536) (end 68.913058 123.879515) (width 0.6) (layer B.Cu) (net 4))
 (segment (start 67.818739 125.817464) (end 67.713058 125.780485) (width 0.6) (layer B.Cu) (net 4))
 (segment (start 70.113058 124.780484) (end 70.018255 124.720915) (width 0.6) (layer B.Cu) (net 4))
 (segment (start 69.546941 123.879515) (end 69.44126 123.842536) (width 0.6) (layer B.Cu) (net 4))
 (segment (start 70.018255 124.720915) (end 69.939084 124.641744) (width 0.6) (layer B.Cu) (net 4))
 (segment (start 68.739084 124.018255) (end 68.679515 124.113058) (width 0.6) (layer B.Cu) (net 4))
 (segment (start 69.879515 124.546941) (end 69.842536 124.44126) (width 0.6) (layer B.Cu) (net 4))
 (segment (start 69.780484 124.113058) (end 69.720915 124.018255) (width 0.6) (layer B.Cu) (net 4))
 (segment (start 68.642536 124.218739) (end 68.63 124.33) (width 0.6) (layer B.Cu) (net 4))
 (segment (start 68.346941 125.780485) (end 68.24126 125.817464) (width 0.6) (layer B.Cu) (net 4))
 (segment (start 70.218739 124.817463) (end 70.113058 124.780484) (width 0.6) (layer B.Cu) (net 4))
 (segment (start 68.63 124.33) (end 68.63 125.33) (width 0.6) (layer B.Cu) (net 4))
 (segment (start 72.7 124.83) (end 70.33 124.83) (width 0.6) (layer B.Cu) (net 4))
 (segment (start 70.33 124.83) (end 70.218739 124.817463) (width 0.6) (layer B.Cu) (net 4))
 (segment (start 69.939084 124.641744) (end 69.879515 124.546941) (width 0.6) (layer B.Cu) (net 4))
 (segment (start 69.13 123.83) (end 69.018739 123.842536) (width 0.6) (layer B.Cu) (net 4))
 (segment (start 68.520915 125.641745) (end 68.441744 125.720916) (width 0.6) (layer B.Cu) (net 4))
 (segment (start 69.817463 124.218739) (end 69.780484 124.113058) (width 0.6) (layer B.Cu) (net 4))
 (segment (start 69.842536 124.44126) (end 69.817463 124.218739) (width 0.6) (layer B.Cu) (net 4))
 (segment (start 67.479515 125.546942) (end 67.442536 125.441261) (width 0.6) (layer B.Cu) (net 4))
 (segment (start 68.617463 125.441261) (end 68.580484 125.546942) (width 0.6) (layer B.Cu) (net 4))
 (segment (start 68.580484 125.546942) (end 68.520915 125.641745) (width 0.6) (layer B.Cu) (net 4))
 (segment (start 68.441744 125.720916) (end 68.346941 125.780485) (width 0.6) (layer B.Cu) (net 4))
 (segment (start 67.146941 123.879515) (end 67.04126 123.842536) (width 0.6) (layer B.Cu) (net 4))
 (segment (start 68.24126 125.817464) (end 68.13 125.83) (width 0.6) (layer B.Cu) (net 4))
 (segment (start 68.13 125.83) (end 67.93 125.83) (width 0.6) (layer B.Cu) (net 4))
 (segment (start 67.618255 125.720916) (end 67.539084 125.641745) (width 0.6) (layer B.Cu) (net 4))
 (segment (start 67.93 125.83) (end 67.818739 125.817464) (width 0.6) (layer B.Cu) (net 4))
 (segment (start 67.713058 125.780485) (end 67.618255 125.720916) (width 0.6) (layer B.Cu) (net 4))
 (segment (start 67.442536 125.441261) (end 67.43 125.33) (width 0.6) (layer B.Cu) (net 4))
 (segment (start 67.43 125.33) (end 67.43 124.33) (width 0.6) (layer B.Cu) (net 4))
 (segment (start 67.320915 124.018255) (end 67.241744 123.939084) (width 0.6) (layer B.Cu) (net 4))
 (segment (start 67.43 124.33) (end 67.417463 124.218739) (width 0.6) (layer B.Cu) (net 4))
 (segment (start 67.417463 124.218739) (end 67.380484 124.113058) (width 0.6) (layer B.Cu) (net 4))
 (segment (start 67.04126 123.842536) (end 66.93 123.83) (width 0.6) (layer B.Cu) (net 4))
 (segment (start 67.380484 124.113058) (end 67.320915 124.018255) (width 0.6) (layer B.Cu) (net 4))
 (segment (start 66.93 123.83) (end 66.73 123.83) (width 0.6) (layer B.Cu) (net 4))
 (segment (start 67.241744 123.939084) (end 67.146941 123.879515) (width 0.6) (layer B.Cu) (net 4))
 (segment (start 72.7 127.37) (end 75.24 127.37) (width 0.6) (layer B.Cu) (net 3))
 (segment (start 72.7 127.37) (end 62.63 127.37) (width 0.6) (layer B.Cu) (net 3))
 (via (at 61 129) (size 1.4) (drill 0.8) (layers F.Cu B.Cu) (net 3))
 (segment (start 62.63 127.37) (end 61 129) (width 0.6) (layer B.Cu) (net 3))
 (segment (start 61 129) (end 61 124.5) (width 0.6) (layer F.Cu) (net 3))
 (via (at 61 124.5) (size 1.4) (drill 0.8) (layers F.Cu B.Cu) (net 3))
 (segment (start 55.47 123.97) (end 38.535 123.97) (width 0.6) (layer B.Cu) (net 3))
 (segment (start 61 124.5) (end 56 124.5) (width 0.6) (layer B.Cu) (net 3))
 (segment (start 56 124.5) (end 55.47 123.97) (width 0.6) (layer B.Cu) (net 3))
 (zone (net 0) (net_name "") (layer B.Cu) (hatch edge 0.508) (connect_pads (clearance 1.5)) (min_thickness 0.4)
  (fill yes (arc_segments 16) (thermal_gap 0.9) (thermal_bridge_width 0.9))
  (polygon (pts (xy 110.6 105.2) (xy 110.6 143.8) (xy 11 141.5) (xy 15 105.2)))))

